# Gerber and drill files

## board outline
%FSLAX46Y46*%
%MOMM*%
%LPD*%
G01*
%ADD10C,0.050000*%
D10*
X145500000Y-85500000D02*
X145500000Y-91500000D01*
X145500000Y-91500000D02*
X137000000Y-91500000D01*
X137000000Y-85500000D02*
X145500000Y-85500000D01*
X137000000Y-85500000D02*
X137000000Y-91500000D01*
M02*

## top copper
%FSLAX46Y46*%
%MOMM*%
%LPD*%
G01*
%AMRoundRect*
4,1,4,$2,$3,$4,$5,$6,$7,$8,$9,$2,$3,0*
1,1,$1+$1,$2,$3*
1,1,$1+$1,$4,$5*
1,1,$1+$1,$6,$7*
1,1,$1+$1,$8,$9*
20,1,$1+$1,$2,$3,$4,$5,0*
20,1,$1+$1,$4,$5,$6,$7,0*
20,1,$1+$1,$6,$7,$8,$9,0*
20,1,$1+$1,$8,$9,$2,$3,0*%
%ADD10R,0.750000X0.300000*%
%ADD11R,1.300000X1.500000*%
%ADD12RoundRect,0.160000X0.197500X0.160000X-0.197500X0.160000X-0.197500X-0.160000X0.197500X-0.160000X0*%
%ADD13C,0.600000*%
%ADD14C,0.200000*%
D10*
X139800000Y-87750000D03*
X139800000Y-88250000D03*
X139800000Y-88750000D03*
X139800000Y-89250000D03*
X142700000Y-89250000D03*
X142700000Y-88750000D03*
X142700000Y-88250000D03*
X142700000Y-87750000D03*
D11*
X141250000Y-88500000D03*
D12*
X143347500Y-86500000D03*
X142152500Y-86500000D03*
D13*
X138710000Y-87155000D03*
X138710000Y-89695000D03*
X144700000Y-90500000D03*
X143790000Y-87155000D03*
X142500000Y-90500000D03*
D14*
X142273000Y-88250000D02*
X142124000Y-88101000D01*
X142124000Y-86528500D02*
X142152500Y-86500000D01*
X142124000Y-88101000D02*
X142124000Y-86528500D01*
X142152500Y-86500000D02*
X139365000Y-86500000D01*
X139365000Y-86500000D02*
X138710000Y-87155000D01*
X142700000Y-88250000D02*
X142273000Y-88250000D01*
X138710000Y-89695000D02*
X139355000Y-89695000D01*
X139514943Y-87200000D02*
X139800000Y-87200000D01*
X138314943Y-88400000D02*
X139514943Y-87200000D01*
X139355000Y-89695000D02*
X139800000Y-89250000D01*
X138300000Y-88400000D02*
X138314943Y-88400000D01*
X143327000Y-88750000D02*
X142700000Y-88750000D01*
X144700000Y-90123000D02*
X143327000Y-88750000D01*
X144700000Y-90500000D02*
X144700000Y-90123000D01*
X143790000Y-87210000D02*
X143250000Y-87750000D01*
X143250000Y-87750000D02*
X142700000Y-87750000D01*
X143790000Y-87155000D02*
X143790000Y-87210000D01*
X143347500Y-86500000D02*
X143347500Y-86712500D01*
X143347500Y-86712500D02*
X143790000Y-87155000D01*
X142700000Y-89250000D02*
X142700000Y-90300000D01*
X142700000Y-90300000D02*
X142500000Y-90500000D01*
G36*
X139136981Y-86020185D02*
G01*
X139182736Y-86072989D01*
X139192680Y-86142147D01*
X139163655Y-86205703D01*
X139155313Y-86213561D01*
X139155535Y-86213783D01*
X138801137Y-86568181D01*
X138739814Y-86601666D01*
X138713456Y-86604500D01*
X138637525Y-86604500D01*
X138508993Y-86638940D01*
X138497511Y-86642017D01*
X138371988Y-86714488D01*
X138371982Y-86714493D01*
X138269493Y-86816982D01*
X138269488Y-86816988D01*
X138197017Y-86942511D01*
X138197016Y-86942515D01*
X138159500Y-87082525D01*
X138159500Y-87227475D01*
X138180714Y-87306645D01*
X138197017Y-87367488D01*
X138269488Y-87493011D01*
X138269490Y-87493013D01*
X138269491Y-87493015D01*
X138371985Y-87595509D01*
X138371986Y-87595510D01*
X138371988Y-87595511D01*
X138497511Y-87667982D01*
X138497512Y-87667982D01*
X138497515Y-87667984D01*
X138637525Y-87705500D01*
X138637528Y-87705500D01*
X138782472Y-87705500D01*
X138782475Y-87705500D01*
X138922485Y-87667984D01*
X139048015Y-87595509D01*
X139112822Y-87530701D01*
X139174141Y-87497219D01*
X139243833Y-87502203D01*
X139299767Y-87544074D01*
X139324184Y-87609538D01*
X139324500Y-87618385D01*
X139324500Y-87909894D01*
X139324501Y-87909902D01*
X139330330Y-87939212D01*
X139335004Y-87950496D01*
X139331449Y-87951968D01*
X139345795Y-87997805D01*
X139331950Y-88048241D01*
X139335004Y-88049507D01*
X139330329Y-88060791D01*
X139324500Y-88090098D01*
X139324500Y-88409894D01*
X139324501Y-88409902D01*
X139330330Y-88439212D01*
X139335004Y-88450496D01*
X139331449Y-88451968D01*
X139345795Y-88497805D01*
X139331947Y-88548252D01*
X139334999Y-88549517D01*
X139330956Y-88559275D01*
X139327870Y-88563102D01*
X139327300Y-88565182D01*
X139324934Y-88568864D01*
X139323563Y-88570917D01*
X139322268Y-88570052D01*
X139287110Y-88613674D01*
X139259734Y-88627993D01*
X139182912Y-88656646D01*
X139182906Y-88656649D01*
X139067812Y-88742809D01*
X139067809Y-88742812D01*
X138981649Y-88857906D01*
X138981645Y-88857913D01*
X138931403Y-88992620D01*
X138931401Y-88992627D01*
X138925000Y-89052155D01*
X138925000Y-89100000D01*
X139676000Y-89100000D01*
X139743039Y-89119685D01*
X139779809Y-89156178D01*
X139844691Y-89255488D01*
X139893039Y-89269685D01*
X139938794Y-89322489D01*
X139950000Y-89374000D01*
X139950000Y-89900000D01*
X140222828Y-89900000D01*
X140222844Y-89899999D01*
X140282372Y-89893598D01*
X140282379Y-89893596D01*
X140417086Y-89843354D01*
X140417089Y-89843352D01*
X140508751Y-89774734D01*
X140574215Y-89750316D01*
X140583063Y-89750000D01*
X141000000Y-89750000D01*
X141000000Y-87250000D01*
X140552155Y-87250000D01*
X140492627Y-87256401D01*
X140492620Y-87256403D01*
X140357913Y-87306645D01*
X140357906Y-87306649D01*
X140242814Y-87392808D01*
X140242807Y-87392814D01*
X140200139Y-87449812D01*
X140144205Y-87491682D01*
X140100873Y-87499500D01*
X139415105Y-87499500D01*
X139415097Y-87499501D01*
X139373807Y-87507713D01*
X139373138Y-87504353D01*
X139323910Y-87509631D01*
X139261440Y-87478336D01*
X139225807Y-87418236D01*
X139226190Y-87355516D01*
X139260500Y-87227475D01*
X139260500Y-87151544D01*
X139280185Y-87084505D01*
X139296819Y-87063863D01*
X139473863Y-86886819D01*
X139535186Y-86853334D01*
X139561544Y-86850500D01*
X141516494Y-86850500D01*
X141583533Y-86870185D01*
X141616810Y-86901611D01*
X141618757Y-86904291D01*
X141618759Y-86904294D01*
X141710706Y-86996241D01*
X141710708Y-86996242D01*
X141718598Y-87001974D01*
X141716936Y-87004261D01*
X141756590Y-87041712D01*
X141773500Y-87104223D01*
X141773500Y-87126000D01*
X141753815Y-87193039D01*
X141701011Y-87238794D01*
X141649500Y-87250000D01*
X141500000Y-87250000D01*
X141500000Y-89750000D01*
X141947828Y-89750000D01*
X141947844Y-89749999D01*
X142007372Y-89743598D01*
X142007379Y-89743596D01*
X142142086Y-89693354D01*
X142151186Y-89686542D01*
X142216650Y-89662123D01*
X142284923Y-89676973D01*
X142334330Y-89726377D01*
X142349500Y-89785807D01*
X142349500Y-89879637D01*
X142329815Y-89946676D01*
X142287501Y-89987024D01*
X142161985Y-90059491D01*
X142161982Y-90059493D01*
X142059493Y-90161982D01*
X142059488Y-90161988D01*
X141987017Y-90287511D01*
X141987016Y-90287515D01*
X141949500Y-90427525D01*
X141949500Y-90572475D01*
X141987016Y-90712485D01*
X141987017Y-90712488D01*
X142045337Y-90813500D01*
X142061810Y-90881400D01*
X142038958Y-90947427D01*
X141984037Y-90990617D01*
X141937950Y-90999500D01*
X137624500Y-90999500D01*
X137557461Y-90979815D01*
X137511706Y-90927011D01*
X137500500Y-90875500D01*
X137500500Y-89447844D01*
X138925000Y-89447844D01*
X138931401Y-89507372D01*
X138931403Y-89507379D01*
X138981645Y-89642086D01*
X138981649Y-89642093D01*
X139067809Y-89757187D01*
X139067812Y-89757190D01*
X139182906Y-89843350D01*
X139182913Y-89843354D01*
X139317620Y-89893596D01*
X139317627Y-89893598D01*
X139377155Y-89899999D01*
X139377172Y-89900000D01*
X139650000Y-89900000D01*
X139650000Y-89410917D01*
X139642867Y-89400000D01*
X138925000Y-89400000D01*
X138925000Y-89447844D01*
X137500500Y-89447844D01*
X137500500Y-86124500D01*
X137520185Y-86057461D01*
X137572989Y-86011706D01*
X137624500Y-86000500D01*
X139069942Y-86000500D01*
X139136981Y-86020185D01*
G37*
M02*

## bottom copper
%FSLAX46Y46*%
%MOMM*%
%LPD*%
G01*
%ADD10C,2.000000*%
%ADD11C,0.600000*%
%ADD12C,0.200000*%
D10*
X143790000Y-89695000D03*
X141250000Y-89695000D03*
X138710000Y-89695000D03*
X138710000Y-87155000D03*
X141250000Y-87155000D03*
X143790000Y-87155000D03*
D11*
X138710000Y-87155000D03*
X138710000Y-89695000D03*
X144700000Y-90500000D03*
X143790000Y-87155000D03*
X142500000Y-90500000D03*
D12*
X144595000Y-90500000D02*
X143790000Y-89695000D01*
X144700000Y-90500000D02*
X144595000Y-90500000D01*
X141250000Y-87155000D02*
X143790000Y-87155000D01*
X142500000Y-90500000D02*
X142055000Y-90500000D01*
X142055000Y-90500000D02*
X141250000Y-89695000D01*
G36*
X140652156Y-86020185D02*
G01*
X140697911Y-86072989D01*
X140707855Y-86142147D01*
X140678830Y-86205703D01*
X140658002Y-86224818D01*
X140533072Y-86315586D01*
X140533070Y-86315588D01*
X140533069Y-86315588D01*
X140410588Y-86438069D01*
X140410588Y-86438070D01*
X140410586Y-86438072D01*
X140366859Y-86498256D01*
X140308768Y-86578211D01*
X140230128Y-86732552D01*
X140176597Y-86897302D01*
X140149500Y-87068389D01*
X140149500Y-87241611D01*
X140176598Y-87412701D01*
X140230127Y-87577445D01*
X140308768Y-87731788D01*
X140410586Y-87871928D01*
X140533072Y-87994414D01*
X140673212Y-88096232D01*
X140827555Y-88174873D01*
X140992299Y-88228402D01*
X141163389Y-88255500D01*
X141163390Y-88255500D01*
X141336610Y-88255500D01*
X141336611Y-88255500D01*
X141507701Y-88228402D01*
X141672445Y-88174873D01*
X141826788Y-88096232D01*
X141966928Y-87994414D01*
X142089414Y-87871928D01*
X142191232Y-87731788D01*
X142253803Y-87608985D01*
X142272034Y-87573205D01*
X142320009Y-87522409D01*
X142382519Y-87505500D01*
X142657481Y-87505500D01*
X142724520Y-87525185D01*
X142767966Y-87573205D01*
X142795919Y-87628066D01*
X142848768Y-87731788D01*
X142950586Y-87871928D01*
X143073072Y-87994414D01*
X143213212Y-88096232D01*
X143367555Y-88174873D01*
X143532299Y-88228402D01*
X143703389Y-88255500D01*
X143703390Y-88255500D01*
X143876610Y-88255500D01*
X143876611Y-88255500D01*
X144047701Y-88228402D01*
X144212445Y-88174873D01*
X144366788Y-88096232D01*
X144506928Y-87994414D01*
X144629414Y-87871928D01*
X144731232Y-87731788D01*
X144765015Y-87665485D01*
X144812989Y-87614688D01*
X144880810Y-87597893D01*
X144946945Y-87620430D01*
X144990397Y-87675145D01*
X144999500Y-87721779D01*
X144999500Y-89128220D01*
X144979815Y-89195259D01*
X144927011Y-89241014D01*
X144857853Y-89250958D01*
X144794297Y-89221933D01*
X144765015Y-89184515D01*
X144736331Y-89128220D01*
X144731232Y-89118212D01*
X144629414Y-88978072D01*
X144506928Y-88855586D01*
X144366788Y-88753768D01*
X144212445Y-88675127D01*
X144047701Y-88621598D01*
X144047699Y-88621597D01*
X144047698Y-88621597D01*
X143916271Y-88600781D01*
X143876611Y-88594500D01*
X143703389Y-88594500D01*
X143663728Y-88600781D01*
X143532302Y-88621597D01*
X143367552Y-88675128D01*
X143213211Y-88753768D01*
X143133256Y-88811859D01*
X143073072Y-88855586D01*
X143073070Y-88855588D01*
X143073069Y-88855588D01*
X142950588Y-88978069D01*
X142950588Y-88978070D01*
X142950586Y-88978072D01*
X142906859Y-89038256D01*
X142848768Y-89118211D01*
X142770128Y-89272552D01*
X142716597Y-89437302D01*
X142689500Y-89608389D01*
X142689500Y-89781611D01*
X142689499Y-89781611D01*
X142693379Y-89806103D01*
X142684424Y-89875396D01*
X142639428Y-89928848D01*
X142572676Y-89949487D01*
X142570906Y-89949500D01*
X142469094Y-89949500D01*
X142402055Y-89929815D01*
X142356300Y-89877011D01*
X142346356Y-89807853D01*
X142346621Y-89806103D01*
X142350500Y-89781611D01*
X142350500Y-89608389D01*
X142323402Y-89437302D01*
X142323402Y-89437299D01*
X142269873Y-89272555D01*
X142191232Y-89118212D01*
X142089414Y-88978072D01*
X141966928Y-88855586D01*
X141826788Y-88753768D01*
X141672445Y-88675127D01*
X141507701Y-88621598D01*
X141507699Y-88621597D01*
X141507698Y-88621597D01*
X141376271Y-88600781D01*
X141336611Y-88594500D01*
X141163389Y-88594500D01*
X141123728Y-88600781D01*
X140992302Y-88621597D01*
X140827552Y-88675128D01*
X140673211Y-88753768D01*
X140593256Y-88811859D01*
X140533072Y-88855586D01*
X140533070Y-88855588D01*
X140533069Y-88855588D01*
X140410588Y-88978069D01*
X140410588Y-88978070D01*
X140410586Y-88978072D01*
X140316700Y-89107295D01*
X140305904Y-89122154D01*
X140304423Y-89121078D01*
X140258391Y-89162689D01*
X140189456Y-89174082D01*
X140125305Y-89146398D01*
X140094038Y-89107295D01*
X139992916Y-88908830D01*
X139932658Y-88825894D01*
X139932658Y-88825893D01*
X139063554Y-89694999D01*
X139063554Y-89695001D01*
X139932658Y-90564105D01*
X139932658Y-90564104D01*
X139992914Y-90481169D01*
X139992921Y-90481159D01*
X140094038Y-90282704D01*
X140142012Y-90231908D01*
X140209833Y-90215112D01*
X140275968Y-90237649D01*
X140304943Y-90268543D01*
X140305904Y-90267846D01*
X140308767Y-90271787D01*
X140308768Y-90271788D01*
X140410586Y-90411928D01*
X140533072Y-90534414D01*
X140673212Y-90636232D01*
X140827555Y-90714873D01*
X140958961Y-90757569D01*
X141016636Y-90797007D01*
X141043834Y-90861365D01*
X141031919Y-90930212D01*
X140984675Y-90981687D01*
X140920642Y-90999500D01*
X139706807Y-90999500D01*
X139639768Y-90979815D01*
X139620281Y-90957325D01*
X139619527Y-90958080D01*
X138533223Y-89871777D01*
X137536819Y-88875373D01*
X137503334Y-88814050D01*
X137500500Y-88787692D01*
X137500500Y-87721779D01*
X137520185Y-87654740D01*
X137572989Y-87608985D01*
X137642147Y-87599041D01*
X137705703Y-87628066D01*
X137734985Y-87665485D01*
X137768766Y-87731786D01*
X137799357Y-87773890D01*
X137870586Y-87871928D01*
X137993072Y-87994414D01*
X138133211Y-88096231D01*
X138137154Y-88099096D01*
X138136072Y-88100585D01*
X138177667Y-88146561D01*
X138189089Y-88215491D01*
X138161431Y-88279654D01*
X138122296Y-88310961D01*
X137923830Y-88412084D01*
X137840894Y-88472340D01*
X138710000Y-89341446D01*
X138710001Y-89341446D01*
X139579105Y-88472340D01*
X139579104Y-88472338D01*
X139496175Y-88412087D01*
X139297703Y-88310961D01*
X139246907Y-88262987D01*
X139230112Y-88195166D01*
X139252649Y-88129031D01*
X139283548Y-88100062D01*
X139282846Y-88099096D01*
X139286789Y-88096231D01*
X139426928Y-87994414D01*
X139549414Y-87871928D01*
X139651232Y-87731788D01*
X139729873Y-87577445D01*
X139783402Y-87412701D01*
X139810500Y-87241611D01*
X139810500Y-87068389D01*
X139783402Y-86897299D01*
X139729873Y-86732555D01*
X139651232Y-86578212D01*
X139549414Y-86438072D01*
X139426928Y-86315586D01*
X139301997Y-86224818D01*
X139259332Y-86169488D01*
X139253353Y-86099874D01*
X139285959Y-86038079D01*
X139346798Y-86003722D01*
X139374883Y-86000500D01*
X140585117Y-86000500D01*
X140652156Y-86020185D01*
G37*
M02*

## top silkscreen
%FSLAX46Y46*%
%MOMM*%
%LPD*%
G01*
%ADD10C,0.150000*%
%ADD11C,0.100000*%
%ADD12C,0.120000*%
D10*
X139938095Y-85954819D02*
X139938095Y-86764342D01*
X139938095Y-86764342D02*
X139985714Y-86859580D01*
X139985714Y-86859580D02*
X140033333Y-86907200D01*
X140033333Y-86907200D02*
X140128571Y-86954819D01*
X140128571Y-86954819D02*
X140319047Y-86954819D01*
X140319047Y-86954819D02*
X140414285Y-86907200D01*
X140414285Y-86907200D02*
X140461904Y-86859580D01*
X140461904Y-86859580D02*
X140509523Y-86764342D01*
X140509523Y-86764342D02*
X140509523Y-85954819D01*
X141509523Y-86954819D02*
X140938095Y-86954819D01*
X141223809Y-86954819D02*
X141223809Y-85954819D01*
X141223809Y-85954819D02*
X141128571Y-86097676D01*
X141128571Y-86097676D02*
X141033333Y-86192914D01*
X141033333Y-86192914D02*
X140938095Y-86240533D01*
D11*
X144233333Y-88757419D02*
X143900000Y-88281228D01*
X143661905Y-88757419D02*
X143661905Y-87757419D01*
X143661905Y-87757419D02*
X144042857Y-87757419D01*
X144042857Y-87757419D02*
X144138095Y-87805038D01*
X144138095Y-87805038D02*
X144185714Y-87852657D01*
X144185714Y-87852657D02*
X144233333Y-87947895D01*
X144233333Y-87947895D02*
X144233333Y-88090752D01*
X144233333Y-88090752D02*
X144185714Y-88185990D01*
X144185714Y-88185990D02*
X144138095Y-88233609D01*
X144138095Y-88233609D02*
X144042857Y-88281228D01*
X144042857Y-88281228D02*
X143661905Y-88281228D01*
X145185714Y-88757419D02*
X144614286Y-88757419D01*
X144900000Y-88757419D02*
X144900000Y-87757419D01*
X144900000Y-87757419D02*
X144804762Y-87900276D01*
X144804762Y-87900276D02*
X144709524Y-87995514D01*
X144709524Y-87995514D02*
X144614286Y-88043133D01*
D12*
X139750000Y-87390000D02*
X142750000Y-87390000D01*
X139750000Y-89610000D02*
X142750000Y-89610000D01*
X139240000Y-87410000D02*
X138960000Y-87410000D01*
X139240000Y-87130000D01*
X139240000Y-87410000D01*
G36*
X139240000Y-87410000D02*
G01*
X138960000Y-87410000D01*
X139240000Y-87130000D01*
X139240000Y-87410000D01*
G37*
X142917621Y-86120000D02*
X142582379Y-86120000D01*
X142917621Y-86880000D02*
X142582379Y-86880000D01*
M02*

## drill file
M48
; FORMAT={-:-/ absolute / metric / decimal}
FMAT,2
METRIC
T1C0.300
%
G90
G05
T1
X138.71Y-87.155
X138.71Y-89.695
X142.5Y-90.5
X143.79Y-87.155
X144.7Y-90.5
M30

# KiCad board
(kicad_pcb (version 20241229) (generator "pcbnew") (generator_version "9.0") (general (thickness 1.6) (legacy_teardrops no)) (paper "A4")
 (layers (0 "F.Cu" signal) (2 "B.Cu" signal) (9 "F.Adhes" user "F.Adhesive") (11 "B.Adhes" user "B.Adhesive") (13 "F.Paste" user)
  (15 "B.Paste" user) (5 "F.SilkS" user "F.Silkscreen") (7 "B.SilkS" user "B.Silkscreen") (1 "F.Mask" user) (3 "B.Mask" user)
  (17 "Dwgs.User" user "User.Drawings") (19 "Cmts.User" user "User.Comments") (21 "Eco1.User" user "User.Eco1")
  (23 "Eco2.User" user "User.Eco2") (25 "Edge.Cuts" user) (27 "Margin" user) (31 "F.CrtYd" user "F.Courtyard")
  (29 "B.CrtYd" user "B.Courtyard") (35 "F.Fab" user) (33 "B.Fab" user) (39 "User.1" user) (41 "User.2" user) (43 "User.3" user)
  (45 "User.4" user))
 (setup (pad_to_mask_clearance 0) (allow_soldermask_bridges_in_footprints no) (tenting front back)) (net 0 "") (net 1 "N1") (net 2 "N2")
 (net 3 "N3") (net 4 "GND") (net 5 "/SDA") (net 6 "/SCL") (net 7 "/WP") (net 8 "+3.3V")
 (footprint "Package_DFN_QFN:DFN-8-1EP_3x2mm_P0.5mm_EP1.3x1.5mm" (layer "F.Cu") (at 141.25 88.5)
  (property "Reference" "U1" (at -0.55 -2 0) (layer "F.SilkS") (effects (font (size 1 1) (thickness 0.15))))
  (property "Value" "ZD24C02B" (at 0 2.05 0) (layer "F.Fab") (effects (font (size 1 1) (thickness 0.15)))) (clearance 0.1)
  (fp_line (start -1.5 -1.11) (end 1.5 -1.11) (stroke (width 0.12) (type solid)) (layer "F.SilkS"))
  (fp_line (start -1.5 1.11) (end 1.5 1.11) (stroke (width 0.12) (type solid)) (layer "F.SilkS"))
  (fp_poly
   (pts (xy -2.01 -1.09) (xy -2.29 -1.09) (xy -2.01 -1.37) (xy -2.01 -1.09)) (stroke (width 0.12) (type solid)) (fill yes) (layer "F.SilkS"))
  (pad "" smd rect (at -0.325 -0.375) (size 0.5 0.6) (layers "F.Paste"))
  (pad "" smd rect (at -0.325 0.375) (size 0.5 0.6) (layers "F.Paste"))
  (pad "" smd rect (at 0.325 -0.375) (size 0.5 0.6) (layers "F.Paste"))
  (pad "" smd rect (at 0.325 0.375) (size 0.5 0.6) (layers "F.Paste"))
  (pad "1" smd rect (at -1.45 -0.75) (size 0.75 0.3) (layers "F.Cu" "F.Mask" "F.Paste") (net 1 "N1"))
  (pad "2" smd rect (at -1.45 -0.25) (size 0.75 0.3) (layers "F.Cu" "F.Mask" "F.Paste") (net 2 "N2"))
  (pad "3" smd rect (at -1.45 0.25) (size 0.75 0.3) (layers "F.Cu" "F.Mask" "F.Paste") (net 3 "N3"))
  (pad "4" smd rect (at -1.45 0.75) (size 0.75 0.3) (layers "F.Cu" "F.Mask" "F.Paste") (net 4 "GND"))
  (pad "5" smd rect (at 1.45 0.75) (size 0.75 0.3) (layers "F.Cu" "F.Mask" "F.Paste") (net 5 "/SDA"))
  (pad "6" smd rect (at 1.45 0.25) (size 0.75 0.3) (layers "F.Cu" "F.Mask" "F.Paste") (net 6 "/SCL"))
  (pad "7" smd rect (at 1.45 -0.25) (size 0.75 0.3) (layers "F.Cu" "F.Mask" "F.Paste") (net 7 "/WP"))
  (pad "8" smd rect (at 1.45 -0.75) (size 0.75 0.3) (layers "F.Cu" "F.Mask" "F.Paste") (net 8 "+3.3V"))
  (pad "9" smd rect (at 0 0) (size 1.3 1.5) (layers "F.Cu" "F.Mask") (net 4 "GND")))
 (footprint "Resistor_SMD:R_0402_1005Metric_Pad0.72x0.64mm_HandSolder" (layer "F.Cu") (at 142.75 86.5 180)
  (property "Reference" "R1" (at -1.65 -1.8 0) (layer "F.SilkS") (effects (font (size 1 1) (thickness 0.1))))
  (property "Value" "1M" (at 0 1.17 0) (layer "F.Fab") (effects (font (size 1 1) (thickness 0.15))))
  (fp_line (start -0.167621 0.38) (end 0.167621 0.38) (stroke (width 0.12) (type solid)) (layer "F.SilkS"))
  (fp_line (start -0.167621 -0.38) (end 0.167621 -0.38) (stroke (width 0.12) (type solid)) (layer "F.SilkS"))
  (pad "1" smd roundrect (at -0.5975 0 180) (size 0.715 0.64) (layers "F.Cu" "F.Mask" "F.Paste") (roundrect_rratio 0.25) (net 8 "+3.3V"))
  (pad "2" smd roundrect (at 0.5975 0 180) (size 0.715 0.64) (layers "F.Cu" "F.Mask" "F.Paste") (roundrect_rratio 0.25) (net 7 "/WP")))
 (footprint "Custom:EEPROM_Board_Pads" (layer "B.Cu") (at 141.25 88.425 180)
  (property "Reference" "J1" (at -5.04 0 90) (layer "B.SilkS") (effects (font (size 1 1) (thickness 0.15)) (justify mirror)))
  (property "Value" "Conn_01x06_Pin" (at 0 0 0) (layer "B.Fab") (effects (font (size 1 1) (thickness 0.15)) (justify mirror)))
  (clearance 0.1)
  (pad "1" smd circle (at -2.54 -1.27 180) (size 2 2) (layers "B.Cu" "B.Mask" "B.Paste") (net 6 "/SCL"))
  (pad "2" smd circle (at 0 -1.27 180) (size 2 2) (layers "B.Cu" "B.Mask" "B.Paste") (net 5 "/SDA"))
  (pad "3" smd circle (at 2.54 -1.27 180) (size 2 2) (layers "B.Cu" "B.Mask" "B.Paste") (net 4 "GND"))
  (pad "4" smd circle (at 2.54 1.27 180) (size 2 2) (layers "B.Cu" "B.Mask" "B.Paste") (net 7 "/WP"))
  (pad "5" smd circle (at 0 1.27 180) (size 2 2) (layers "B.Cu" "B.Mask" "B.Paste") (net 8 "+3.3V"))
  (pad "6" smd circle (at -2.54 1.27 180) (size 2 2) (layers "B.Cu" "B.Mask" "B.Paste") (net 8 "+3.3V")))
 (gr_line (start 145.5 85.5) (end 145.5 91.5) (stroke (width 0.05) (type default)) (layer "Edge.Cuts"))
 (gr_line (start 145.5 91.5) (end 137 91.5) (stroke (width 0.05) (type default)) (layer "Edge.Cuts"))
 (gr_line (start 137 85.5) (end 145.5 85.5) (stroke (width 0.05) (type default)) (layer "Edge.Cuts"))
 (gr_line (start 137 85.5) (end 137 91.5) (stroke (width 0.05) (type default)) (layer "Edge.Cuts"))
 (segment (start 142.273 88.25) (end 142.124 88.101) (width 0.2) (layer "F.Cu") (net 7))
 (segment (start 142.124 86.5285) (end 142.1525 86.5) (width 0.2) (layer "F.Cu") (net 7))
 (segment (start 142.124 88.101) (end 142.124 86.5285) (width 0.2) (layer "F.Cu") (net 7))
 (segment (start 142.1525 86.5) (end 139.365 86.5) (width 0.2) (layer "F.Cu") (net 7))
 (segment (start 139.365 86.5) (end 138.71 87.155) (width 0.2) (layer "F.Cu") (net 7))
 (segment (start 142.7 88.25) (end 142.273 88.25) (width 0.2) (layer "F.Cu") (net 7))
 (via (at 138.71 87.155) (size 0.6) (drill 0.3) (layers "F.Cu" "B.Cu") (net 7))
 (segment (start 138.71 89.695) (end 139.355 89.695) (width 0.2) (layer "F.Cu") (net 4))
 (segment (start 139.514943 87.2) (end 139.8 87.2) (width 0.2) (layer "F.Cu") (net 4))
 (segment (start 138.314943 88.4) (end 139.514943 87.2) (width 0.2) (layer "F.Cu") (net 4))
 (segment (start 139.355 89.695) (end 139.8 89.25) (width 0.2) (layer "F.Cu") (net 4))
 (segment (start 138.3 88.4) (end 138.314943 88.4) (width 0.2) (layer "F.Cu") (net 4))
 (via (at 138.71 89.695) (size 0.6) (drill 0.3) (layers "F.Cu" "B.Cu") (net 4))
 (segment (start 143.327 88.75) (end 142.7 88.75) (width 0.2) (layer "F.Cu") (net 6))
 (segment (start 144.7 90.123) (end 143.327 88.75) (width 0.2) (layer "F.Cu") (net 6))
 (segment (start 144.7 90.5) (end 144.7 90.123) (width 0.2) (layer "F.Cu") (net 6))
 (via (at 144.7 90.5) (size 0.6) (drill 0.3) (layers "F.Cu" "B.Cu") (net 6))
 (segment (start 144.595 90.5) (end 143.79 89.695) (width 0.2) (layer "B.Cu") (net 6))
 (segment (start 144.7 90.5) (end 144.595 90.5) (width 0.2) (layer "B.Cu") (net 6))
 (segment (start 143.79 87.21) (end 143.25 87.75) (width 0.2) (layer "F.Cu") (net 8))
 (segment (start 143.25 87.75) (end 142.7 87.75) (width 0.2) (layer "F.Cu") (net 8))
 (segment (start 143.79 87.155) (end 143.79 87.21) (width 0.2) (layer "F.Cu") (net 8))
 (segment (start 143.3475 86.5) (end 143.3475 86.7125) (width 0.2) (layer "F.Cu") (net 8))
 (segment (start 143.3475 86.7125) (end 143.79 87.155) (width 0.2) (layer "F.Cu") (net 8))
 (via (at 143.79 87.155) (size 0.6) (drill 0.3) (layers "F.Cu" "B.Cu") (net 8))
 (segment (start 141.25 87.155) (end 143.79 87.155) (width 0.2) (layer "B.Cu") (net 8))
 (segment (start 142.7 89.25) (end 142.7 90.3) (width 0.2) (layer "F.Cu") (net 5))
 (segment (start 142.7 90.3) (end 142.5 90.5) (width 0.2) (layer "F.Cu") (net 5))
 (via (at 142.5 90.5) (size 0.6) (drill 0.3) (layers "F.Cu" "B.Cu") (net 5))
 (segment (start 142.5 90.5) (end 142.055 90.5) (width 0.2) (layer "B.Cu") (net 5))
 (segment (start 142.055 90.5) (end 141.25 89.695) (width 0.2) (layer "B.Cu") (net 5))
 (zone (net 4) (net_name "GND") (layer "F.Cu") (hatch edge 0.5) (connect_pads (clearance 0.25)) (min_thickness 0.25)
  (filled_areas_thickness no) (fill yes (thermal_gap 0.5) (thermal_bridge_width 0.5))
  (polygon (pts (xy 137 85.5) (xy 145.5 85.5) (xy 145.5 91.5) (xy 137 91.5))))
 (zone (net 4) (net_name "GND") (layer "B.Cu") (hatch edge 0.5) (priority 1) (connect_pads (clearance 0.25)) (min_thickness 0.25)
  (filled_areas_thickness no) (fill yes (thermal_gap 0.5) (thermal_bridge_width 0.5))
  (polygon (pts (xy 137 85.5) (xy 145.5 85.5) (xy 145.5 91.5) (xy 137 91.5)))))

